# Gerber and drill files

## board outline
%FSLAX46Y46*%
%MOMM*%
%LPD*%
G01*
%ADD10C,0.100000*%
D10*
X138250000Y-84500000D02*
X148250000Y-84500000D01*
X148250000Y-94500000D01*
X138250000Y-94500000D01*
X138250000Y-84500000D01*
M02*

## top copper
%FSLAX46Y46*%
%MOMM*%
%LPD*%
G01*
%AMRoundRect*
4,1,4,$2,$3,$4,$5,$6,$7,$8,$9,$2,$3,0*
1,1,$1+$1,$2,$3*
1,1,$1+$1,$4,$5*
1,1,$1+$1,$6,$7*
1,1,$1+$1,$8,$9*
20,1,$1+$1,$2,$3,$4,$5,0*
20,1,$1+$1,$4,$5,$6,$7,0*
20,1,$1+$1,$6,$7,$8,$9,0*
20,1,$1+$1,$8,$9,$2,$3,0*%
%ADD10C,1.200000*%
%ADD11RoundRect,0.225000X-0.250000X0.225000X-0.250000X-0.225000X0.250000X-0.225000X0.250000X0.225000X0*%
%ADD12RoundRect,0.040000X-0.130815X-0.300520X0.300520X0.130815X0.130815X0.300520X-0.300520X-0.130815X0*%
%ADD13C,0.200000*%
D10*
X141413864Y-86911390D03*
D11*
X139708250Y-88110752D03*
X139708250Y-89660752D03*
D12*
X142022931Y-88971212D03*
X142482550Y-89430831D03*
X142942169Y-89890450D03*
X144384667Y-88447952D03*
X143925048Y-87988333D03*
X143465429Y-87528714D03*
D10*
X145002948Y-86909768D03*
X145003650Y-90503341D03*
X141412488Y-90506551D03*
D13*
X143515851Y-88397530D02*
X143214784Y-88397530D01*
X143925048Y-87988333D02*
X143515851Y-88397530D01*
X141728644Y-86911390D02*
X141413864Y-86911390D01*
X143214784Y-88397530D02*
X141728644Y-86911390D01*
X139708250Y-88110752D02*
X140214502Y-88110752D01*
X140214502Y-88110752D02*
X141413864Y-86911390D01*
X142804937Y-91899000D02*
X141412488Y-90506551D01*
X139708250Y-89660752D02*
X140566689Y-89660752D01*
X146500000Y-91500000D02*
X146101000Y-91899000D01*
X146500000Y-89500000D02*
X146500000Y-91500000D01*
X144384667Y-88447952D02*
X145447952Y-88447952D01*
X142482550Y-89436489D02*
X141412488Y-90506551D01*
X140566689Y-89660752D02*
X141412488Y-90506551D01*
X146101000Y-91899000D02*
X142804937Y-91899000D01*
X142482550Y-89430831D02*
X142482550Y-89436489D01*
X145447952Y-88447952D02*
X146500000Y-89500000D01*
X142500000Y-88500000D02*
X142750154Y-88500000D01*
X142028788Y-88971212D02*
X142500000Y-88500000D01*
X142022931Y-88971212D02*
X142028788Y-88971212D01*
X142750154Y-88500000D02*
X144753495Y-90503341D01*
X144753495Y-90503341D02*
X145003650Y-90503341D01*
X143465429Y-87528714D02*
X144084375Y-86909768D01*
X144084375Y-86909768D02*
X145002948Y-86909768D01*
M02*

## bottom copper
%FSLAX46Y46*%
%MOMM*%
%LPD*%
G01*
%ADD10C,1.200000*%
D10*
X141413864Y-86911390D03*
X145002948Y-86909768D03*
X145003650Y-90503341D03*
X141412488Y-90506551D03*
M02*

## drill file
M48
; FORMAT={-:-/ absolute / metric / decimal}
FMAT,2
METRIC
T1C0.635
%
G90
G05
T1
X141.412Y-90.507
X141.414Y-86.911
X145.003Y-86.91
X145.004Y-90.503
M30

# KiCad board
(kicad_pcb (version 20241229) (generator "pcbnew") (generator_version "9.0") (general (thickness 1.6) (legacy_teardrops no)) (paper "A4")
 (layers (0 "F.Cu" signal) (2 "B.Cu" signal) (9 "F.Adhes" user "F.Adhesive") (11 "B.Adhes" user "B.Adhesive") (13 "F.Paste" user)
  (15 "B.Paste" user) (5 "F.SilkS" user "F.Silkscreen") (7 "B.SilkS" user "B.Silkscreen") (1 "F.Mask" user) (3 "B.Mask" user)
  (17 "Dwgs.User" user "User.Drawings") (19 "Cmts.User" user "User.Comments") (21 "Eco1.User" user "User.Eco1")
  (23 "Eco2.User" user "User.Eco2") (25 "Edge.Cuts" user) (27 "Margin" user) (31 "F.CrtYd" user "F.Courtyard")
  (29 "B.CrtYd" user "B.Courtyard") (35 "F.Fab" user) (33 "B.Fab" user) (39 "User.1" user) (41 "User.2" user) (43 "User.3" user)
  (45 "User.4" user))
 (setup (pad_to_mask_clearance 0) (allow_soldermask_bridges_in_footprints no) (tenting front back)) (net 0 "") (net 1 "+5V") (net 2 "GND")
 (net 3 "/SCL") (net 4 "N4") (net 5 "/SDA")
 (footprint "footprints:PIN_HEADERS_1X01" (layer "F.Cu") (at 141.413864 86.91139)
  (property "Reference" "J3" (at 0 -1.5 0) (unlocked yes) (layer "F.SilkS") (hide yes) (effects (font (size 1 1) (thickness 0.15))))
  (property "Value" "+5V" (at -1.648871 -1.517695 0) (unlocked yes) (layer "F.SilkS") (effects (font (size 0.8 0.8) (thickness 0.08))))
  (pad "1" thru_hole circle (at 0 0) (size 1.2 1.2) (drill 0.635) (layers "*.Cu" "*.Mask") (remove_unused_layers no) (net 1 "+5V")))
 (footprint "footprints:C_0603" (layer "F.Cu") (at 139.70825 88.885752 -90)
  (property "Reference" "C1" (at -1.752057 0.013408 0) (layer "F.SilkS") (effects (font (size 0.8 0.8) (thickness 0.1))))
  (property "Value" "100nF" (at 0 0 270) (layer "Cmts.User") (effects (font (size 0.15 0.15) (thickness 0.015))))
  (pad "1" smd roundrect (at -0.775 0 270) (size 0.9 0.95) (layers "F.Cu" "F.Mask" "F.Paste") (roundrect_rratio 0.25) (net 1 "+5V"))
  (pad "2" smd roundrect (at 0.775 0 270) (size 0.9 0.95) (layers "F.Cu" "F.Mask" "F.Paste") (roundrect_rratio 0.25) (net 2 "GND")))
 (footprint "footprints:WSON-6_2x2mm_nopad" (layer "F.Cu") (at 143.203799 88.709582 45)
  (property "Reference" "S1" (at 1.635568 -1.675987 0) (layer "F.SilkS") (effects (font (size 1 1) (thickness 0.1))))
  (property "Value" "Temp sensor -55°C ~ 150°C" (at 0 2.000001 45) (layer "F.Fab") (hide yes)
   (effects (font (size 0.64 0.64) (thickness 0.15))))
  (pad "1" smd roundrect (at -1.02 -0.649999 45) (size 0.69 0.32) (layers "F.Cu" "F.Mask" "F.Paste") (roundrect_rratio 0.125) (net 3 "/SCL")
   (solder_mask_margin 0.102))
  (pad "2" smd roundrect (at -1.02 0 45) (size 0.69 0.32) (layers "F.Cu" "F.Mask" "F.Paste") (roundrect_rratio 0.125) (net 2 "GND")
   (solder_mask_margin 0.102))
  (pad "3" smd roundrect (at -1.02 0.649999 45) (size 0.69 0.32) (layers "F.Cu" "F.Mask" "F.Paste") (roundrect_rratio 0.125) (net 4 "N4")
   (solder_mask_margin 0.102))
  (pad "4" smd roundrect (at 1.02 0.649999 45) (size 0.69 0.32) (layers "F.Cu" "F.Mask" "F.Paste") (roundrect_rratio 0.125) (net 2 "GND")
   (solder_mask_margin 0.102))
  (pad "5" smd roundrect (at 1.02 0 45) (size 0.69 0.32) (layers "F.Cu" "F.Mask" "F.Paste") (roundrect_rratio 0.125) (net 1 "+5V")
   (solder_mask_margin 0.102))
  (pad "6" smd roundrect (at 1.02 -0.649999 45) (size 0.69 0.32) (layers "F.Cu" "F.Mask" "F.Paste") (roundrect_rratio 0.125) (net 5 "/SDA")
   (solder_mask_margin 0.102)))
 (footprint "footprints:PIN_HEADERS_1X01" (layer "F.Cu") (at 145.002948 86.909768)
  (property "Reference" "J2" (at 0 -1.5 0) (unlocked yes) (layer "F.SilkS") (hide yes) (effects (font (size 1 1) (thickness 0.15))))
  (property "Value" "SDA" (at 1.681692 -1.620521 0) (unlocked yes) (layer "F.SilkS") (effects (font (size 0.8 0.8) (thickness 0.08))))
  (pad "1" thru_hole circle (at 0 0) (size 1.2 1.2) (drill 0.635) (layers "*.Cu" "*.Mask") (remove_unused_layers no) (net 5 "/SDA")))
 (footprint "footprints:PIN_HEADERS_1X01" (layer "F.Cu") (at 145.00365 90.503341)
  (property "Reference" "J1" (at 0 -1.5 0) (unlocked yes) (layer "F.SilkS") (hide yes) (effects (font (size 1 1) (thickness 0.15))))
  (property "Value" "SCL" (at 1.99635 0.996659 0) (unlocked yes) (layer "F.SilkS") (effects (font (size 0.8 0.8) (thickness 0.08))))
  (pad "1" thru_hole circle (at 0 0) (size 1.2 1.2) (drill 0.635) (layers "*.Cu" "*.Mask") (remove_unused_layers no) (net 3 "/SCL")))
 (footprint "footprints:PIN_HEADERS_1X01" (layer "F.Cu") (at 141.412488 90.506551)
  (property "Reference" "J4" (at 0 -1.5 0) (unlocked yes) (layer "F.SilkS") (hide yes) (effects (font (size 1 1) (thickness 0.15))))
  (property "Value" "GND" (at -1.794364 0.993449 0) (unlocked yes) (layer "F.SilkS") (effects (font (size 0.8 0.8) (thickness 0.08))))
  (pad "1" thru_hole circle (at 0 0) (size 1.2 1.2) (drill 0.635) (layers "*.Cu" "*.Mask") (remove_unused_layers no) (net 2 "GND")))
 (gr_rect (start 138.25 84.5) (end 148.25 94.5) (stroke (width 0.1) (type solid)) (fill no) (layer "Edge.Cuts"))
 (segment (start 143.515851 88.39753) (end 143.214784 88.39753) (width 0.2) (layer "F.Cu") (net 1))
 (segment (start 143.925048 87.988333) (end 143.515851 88.39753) (width 0.2) (layer "F.Cu") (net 1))
 (segment (start 141.728644 86.91139) (end 141.413864 86.91139) (width 0.2) (layer "F.Cu") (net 1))
 (segment (start 143.214784 88.39753) (end 141.728644 86.91139) (width 0.2) (layer "F.Cu") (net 1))
 (segment (start 139.70825 88.110752) (end 140.214502 88.110752) (width 0.2) (layer "F.Cu") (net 1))
 (segment (start 140.214502 88.110752) (end 141.413864 86.91139) (width 0.2) (layer "F.Cu") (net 1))
 (segment (start 142.804937 91.899) (end 141.412488 90.506551) (width 0.2) (layer "F.Cu") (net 2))
 (segment (start 139.70825 89.660752) (end 140.566689 89.660752) (width 0.2) (layer "F.Cu") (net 2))
 (segment (start 146.5 91.5) (end 146.101 91.899) (width 0.2) (layer "F.Cu") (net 2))
 (segment (start 146.5 89.5) (end 146.5 91.5) (width 0.2) (layer "F.Cu") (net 2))
 (segment (start 144.384667 88.447952) (end 145.447952 88.447952) (width 0.2) (layer "F.Cu") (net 2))
 (segment (start 142.48255 89.436489) (end 141.412488 90.506551) (width 0.2) (layer "F.Cu") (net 2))
 (segment (start 140.566689 89.660752) (end 141.412488 90.506551) (width 0.2) (layer "F.Cu") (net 2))
 (segment (start 146.101 91.899) (end 142.804937 91.899) (width 0.2) (layer "F.Cu") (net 2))
 (segment (start 142.48255 89.430831) (end 142.48255 89.436489) (width 0.2) (layer "F.Cu") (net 2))
 (segment (start 145.447952 88.447952) (end 146.5 89.5) (width 0.2) (layer "F.Cu") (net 2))
 (segment (start 142.5 88.5) (end 142.750154 88.5) (width 0.2) (layer "F.Cu") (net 3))
 (segment (start 142.028788 88.971212) (end 142.5 88.5) (width 0.2) (layer "F.Cu") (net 3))
 (segment (start 142.022931 88.971212) (end 142.028788 88.971212) (width 0.2) (layer "F.Cu") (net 3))
 (segment (start 142.750154 88.5) (end 144.753495 90.503341) (width 0.2) (layer "F.Cu") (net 3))
 (segment (start 144.753495 90.503341) (end 145.00365 90.503341) (width 0.2) (layer "F.Cu") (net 3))
 (segment (start 143.465429 87.528714) (end 144.084375 86.909768) (width 0.2) (layer "F.Cu") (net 5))
 (segment (start 144.084375 86.909768) (end 145.002948 86.909768) (width 0.2) (layer "F.Cu") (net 5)))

